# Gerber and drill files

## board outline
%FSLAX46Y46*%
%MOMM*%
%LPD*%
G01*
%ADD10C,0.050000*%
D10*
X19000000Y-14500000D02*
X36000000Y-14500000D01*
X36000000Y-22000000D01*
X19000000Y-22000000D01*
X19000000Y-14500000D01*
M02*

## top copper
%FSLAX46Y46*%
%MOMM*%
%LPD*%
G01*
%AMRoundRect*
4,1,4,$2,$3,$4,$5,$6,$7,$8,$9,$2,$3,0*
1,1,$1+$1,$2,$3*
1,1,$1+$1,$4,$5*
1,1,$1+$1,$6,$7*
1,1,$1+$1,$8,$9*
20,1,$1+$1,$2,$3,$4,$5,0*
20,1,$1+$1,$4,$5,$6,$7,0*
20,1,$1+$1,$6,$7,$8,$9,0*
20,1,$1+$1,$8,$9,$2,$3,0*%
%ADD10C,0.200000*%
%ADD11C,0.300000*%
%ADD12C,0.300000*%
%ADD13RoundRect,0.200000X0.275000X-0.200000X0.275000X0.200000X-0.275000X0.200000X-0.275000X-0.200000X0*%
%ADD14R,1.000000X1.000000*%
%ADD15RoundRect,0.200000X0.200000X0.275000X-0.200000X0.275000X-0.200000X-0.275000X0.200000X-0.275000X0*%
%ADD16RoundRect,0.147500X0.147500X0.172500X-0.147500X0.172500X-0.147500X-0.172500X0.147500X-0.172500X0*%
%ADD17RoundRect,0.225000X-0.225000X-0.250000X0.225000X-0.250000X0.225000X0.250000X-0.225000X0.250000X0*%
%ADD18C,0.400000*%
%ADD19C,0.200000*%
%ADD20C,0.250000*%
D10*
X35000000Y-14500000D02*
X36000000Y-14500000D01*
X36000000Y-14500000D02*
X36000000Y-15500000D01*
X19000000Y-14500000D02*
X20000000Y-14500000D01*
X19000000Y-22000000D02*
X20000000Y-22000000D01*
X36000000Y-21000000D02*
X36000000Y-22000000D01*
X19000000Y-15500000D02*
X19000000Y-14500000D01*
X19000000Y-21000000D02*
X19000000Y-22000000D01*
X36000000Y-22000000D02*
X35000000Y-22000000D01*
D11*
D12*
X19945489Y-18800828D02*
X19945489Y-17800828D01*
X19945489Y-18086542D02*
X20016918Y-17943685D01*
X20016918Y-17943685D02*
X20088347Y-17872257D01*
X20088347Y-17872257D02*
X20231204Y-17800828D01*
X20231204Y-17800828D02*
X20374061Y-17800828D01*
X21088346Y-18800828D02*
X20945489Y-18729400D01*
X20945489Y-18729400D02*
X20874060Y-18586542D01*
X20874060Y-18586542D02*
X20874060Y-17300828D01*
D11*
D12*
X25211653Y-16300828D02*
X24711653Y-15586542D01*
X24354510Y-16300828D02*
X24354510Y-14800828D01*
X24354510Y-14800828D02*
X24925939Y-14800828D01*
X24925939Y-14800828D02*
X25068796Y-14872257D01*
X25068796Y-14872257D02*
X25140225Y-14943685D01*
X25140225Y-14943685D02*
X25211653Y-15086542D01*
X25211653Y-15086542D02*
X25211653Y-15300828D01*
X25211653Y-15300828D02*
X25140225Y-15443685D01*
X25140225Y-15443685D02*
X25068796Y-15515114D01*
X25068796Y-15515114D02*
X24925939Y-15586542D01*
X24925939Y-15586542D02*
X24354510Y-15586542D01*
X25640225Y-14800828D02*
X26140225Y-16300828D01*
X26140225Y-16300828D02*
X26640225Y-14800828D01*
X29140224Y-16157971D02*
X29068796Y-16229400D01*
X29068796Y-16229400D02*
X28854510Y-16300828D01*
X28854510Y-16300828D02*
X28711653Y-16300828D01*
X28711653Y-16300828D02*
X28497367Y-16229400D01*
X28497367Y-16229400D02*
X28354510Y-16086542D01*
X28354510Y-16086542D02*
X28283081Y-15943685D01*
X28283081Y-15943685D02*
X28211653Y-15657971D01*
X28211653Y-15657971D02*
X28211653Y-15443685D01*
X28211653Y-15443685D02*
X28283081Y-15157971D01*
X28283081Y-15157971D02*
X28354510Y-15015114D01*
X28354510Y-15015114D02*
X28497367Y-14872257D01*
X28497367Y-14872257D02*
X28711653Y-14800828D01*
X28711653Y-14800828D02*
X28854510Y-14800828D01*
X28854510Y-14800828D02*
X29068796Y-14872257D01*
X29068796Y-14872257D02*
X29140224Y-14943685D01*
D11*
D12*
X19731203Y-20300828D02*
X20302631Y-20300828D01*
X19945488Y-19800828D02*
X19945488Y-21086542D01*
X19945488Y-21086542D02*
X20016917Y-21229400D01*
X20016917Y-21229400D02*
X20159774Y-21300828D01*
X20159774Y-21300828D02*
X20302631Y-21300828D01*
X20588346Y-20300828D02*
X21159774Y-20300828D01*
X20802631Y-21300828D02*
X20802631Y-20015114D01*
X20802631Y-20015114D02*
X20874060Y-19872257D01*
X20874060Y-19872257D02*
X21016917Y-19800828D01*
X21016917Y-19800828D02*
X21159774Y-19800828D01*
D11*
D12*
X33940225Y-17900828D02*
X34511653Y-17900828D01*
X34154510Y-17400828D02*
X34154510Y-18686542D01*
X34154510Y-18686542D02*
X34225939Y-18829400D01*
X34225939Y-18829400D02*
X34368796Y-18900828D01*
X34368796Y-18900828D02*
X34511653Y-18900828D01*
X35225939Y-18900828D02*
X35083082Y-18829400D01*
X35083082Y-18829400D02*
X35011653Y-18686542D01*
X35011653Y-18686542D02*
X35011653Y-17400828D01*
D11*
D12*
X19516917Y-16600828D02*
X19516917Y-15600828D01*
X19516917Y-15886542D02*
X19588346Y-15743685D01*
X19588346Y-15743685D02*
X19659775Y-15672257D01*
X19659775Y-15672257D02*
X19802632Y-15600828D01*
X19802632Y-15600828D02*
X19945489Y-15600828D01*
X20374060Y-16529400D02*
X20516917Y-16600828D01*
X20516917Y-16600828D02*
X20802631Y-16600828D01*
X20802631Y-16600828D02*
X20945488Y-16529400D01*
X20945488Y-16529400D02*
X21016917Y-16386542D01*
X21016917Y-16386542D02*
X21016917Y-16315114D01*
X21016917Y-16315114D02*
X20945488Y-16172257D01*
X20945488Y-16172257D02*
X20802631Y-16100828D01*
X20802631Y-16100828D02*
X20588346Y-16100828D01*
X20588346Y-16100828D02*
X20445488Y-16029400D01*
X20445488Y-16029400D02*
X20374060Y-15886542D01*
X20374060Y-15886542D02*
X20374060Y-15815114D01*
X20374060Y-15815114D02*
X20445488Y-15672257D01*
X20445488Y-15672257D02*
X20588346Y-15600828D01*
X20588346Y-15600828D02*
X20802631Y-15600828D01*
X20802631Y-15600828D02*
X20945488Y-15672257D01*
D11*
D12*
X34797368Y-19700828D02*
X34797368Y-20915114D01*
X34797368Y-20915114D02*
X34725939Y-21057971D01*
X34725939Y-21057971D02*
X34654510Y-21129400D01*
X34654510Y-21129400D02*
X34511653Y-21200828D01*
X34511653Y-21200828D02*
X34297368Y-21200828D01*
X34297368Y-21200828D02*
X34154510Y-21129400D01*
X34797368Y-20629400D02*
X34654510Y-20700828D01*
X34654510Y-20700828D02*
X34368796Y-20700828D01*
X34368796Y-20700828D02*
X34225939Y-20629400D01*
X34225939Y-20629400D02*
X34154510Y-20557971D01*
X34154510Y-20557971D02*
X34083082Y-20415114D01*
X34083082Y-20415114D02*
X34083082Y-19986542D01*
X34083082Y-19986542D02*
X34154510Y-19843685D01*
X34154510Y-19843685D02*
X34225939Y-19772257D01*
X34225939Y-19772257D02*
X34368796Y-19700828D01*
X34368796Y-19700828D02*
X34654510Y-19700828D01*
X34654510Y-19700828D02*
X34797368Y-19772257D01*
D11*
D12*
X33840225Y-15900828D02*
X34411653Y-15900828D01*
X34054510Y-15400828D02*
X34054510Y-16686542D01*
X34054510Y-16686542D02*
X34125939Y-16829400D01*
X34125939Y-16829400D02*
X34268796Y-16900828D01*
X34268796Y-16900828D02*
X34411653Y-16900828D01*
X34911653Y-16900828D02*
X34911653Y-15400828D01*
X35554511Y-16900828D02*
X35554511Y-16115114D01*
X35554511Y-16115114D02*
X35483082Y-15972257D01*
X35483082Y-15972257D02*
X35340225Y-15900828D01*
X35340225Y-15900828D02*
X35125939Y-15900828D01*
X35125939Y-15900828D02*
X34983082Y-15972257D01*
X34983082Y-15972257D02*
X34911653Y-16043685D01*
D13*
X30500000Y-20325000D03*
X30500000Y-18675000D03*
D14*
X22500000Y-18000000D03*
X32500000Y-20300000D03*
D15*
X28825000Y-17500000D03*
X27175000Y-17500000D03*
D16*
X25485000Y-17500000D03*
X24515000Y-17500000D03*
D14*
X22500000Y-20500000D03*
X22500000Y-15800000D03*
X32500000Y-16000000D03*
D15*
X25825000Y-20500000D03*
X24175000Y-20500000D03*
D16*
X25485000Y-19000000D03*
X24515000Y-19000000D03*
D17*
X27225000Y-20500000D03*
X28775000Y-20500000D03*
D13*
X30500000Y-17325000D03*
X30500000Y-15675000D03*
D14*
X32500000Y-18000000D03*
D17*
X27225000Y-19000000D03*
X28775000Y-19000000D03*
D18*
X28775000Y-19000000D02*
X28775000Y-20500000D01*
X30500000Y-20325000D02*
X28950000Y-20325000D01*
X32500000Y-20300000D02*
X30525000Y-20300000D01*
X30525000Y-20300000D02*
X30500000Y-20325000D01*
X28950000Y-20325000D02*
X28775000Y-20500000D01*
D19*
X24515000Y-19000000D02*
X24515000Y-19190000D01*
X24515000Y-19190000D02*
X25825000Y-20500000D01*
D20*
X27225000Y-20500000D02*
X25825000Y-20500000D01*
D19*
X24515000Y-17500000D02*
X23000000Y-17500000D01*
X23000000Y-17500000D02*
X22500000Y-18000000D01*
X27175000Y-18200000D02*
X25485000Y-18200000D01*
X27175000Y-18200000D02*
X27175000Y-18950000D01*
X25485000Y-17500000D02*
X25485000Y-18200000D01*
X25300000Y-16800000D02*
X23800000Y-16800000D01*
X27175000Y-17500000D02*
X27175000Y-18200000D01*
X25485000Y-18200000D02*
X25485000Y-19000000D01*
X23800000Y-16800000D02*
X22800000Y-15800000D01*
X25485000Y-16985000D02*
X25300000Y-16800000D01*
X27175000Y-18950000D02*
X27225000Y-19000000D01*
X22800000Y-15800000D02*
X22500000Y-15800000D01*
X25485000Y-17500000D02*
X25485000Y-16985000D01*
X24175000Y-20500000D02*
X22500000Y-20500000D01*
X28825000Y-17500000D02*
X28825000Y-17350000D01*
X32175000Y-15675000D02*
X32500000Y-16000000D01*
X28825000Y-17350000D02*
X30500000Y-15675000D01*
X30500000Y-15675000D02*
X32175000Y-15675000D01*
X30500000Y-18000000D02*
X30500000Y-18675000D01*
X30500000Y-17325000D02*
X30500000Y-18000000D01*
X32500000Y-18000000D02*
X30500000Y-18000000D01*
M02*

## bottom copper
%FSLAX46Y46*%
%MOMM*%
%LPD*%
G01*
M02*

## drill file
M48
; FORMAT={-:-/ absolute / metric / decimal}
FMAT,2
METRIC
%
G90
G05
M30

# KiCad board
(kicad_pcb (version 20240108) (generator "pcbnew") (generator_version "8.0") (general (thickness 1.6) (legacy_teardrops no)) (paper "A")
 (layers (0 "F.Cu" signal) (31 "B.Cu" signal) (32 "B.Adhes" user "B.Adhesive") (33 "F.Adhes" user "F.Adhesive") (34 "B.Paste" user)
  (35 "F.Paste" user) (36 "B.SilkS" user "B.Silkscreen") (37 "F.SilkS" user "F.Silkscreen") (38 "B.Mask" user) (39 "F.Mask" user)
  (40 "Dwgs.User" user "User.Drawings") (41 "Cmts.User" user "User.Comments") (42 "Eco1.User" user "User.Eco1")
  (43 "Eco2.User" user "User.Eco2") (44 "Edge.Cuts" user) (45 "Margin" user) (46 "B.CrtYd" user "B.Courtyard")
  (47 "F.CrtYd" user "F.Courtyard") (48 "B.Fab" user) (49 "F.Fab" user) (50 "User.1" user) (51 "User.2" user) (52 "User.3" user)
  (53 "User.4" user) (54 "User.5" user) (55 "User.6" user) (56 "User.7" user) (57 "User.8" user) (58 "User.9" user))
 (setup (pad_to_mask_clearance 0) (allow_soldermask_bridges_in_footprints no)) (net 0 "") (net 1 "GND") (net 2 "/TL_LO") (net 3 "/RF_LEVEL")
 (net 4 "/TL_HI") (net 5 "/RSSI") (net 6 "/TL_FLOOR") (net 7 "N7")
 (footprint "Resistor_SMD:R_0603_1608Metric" (layer "F.Cu") (at 30.5 19.5 90)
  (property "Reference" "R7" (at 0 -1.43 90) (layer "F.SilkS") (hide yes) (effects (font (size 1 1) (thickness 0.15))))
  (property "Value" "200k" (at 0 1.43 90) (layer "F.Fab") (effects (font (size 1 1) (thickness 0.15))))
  (pad "1" smd roundrect (at -0.825 0 90) (size 0.8 0.95) (layers "F.Cu" "F.Paste" "F.Mask") (roundrect_rratio 0.25) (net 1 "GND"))
  (pad "2" smd roundrect (at 0.825 0 90) (size 0.8 0.95) (layers "F.Cu" "F.Paste" "F.Mask") (roundrect_rratio 0.25) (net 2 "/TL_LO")))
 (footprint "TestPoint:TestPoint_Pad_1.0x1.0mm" (layer "F.Cu") (at 22.5 18)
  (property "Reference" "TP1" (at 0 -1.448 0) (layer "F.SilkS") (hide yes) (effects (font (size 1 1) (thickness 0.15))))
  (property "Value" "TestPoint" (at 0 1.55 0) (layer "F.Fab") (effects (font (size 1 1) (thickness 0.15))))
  (pad "1" smd rect (at 0 0) (size 1 1) (layers "F.Cu" "F.Mask") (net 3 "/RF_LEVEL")))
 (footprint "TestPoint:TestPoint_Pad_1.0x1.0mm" (layer "F.Cu") (at 32.5 20.3 90)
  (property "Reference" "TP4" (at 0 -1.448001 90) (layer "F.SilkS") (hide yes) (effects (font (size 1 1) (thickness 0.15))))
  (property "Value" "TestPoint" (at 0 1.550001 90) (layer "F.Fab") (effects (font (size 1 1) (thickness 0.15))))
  (pad "1" smd rect (at 0 0 90) (size 1 1) (layers "F.Cu" "F.Mask") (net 1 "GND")))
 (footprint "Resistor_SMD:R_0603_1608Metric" (layer "F.Cu") (at 28 17.5 180)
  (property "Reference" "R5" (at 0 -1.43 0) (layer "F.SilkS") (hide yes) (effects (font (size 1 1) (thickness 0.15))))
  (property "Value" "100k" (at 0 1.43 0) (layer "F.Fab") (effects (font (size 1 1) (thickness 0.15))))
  (pad "1" smd roundrect (at -0.825 0 180) (size 0.8 0.95) (layers "F.Cu" "F.Paste" "F.Mask") (roundrect_rratio 0.25) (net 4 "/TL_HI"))
  (pad "2" smd roundrect (at 0.825 0 180) (size 0.8 0.95) (layers "F.Cu" "F.Paste" "F.Mask") (roundrect_rratio 0.25) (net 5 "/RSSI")))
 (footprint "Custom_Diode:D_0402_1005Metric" (layer "F.Cu") (at 25 17.5 180)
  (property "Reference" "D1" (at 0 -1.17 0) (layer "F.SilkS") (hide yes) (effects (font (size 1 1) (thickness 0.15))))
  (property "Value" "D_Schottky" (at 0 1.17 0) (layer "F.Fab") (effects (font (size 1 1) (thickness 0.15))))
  (pad "1" smd roundrect (at -0.485 0 180) (size 0.59 0.64) (layers "F.Cu" "F.Paste" "F.Mask") (roundrect_rratio 0.25) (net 5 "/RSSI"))
  (pad "2" smd roundrect (at 0.485 0 180) (size 0.59 0.64) (layers "F.Cu" "F.Paste" "F.Mask") (roundrect_rratio 0.25) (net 3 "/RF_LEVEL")))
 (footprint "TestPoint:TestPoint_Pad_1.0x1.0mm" (layer "F.Cu") (at 22.5 20.5)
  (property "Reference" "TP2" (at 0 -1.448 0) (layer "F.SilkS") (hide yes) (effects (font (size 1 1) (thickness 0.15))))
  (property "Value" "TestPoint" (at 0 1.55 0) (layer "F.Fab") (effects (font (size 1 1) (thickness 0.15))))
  (pad "1" smd rect (at 0 0) (size 1 1) (layers "F.Cu" "F.Mask") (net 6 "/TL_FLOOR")))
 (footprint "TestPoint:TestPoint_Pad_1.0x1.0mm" (layer "F.Cu") (at 22.5 15.8)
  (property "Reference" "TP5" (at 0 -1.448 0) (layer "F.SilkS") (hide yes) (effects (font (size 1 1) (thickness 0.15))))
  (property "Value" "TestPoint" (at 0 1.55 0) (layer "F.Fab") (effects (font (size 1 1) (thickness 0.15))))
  (pad "1" smd rect (at 0 0) (size 1 1) (layers "F.Cu" "F.Mask") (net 5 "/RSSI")))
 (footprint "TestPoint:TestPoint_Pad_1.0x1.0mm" (layer "F.Cu") (at 32.5 16)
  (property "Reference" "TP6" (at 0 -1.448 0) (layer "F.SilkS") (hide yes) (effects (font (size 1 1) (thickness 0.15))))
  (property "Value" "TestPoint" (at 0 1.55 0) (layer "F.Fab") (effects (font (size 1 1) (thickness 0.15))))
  (pad "1" smd rect (at 0 0) (size 1 1) (layers "F.Cu" "F.Mask") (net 4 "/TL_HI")))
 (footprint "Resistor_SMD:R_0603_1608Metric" (layer "F.Cu") (at 25 20.5 180)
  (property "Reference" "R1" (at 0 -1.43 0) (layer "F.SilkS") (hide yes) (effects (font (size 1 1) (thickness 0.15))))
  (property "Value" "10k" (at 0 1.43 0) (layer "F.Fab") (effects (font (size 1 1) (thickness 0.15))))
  (pad "1" smd roundrect (at -0.825 0 180) (size 0.8 0.95) (layers "F.Cu" "F.Paste" "F.Mask") (roundrect_rratio 0.25) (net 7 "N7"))
  (pad "2" smd roundrect (at 0.825 0 180) (size 0.8 0.95) (layers "F.Cu" "F.Paste" "F.Mask") (roundrect_rratio 0.25) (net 6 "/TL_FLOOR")))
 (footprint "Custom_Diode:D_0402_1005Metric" (layer "F.Cu") (at 25 19 180)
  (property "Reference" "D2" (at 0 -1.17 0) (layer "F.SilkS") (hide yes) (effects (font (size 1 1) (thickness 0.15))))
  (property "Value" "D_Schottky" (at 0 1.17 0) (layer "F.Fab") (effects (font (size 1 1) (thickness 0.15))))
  (pad "1" smd roundrect (at -0.485 0 180) (size 0.59 0.64) (layers "F.Cu" "F.Paste" "F.Mask") (roundrect_rratio 0.25) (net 5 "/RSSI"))
  (pad "2" smd roundrect (at 0.485 0 180) (size 0.59 0.64) (layers "F.Cu" "F.Paste" "F.Mask") (roundrect_rratio 0.25) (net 7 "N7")))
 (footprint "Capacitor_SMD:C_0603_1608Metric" (layer "F.Cu") (at 28 20.5)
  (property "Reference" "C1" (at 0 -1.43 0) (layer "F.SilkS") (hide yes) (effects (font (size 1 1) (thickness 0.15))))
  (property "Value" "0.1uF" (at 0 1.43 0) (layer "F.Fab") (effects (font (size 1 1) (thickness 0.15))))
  (pad "1" smd roundrect (at -0.775 0) (size 0.9 0.95) (layers "F.Cu" "F.Paste" "F.Mask") (roundrect_rratio 0.25) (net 7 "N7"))
  (pad "2" smd roundrect (at 0.775 0) (size 0.9 0.95) (layers "F.Cu" "F.Paste" "F.Mask") (roundrect_rratio 0.25) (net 1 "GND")))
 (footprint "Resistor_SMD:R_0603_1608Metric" (layer "F.Cu") (at 30.5 16.5 90)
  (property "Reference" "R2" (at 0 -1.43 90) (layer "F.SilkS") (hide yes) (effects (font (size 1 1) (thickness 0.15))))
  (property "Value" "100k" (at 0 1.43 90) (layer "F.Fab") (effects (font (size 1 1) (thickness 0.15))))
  (pad "1" smd roundrect (at -0.825 0 90) (size 0.8 0.95) (layers "F.Cu" "F.Paste" "F.Mask") (roundrect_rratio 0.25) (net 2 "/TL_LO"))
  (pad "2" smd roundrect (at 0.825 0 90) (size 0.8 0.95) (layers "F.Cu" "F.Paste" "F.Mask") (roundrect_rratio 0.25) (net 4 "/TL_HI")))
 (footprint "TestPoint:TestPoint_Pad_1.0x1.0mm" (layer "F.Cu") (at 32.5 18)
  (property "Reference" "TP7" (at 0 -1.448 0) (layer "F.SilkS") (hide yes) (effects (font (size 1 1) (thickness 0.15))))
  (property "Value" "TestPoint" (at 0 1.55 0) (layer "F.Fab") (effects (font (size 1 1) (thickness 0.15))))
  (pad "1" smd rect (at 0 0) (size 1 1) (layers "F.Cu" "F.Mask") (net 2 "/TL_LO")))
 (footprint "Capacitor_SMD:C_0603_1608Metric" (layer "F.Cu") (at 28 19)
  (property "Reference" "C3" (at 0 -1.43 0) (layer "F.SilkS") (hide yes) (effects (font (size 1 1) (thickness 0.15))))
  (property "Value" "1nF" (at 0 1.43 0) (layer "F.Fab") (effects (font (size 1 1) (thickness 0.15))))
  (pad "1" smd roundrect (at -0.775 0) (size 0.9 0.95) (layers "F.Cu" "F.Paste" "F.Mask") (roundrect_rratio 0.25) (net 5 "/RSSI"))
  (pad "2" smd roundrect (at 0.775 0) (size 0.9 0.95) (layers "F.Cu" "F.Paste" "F.Mask") (roundrect_rratio 0.25) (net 1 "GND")))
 (gr_line (start 35 14.5) (end 36 14.5) (stroke (width 0.2) (type default)) (layer "F.Cu"))
 (gr_line (start 36 14.5) (end 36 15.5) (stroke (width 0.2) (type default)) (layer "F.Cu"))
 (gr_line (start 19 14.5) (end 20 14.5) (stroke (width 0.2) (type default)) (layer "F.Cu"))
 (gr_line (start 19 22) (end 20 22) (stroke (width 0.2) (type default)) (layer "F.Cu"))
 (gr_line (start 36 21) (end 36 22) (stroke (width 0.2) (type default)) (layer "F.Cu"))
 (gr_line (start 19 15.5) (end 19 14.5) (stroke (width 0.2) (type default)) (layer "F.Cu"))
 (gr_line (start 19 21) (end 19 22) (stroke (width 0.2) (type default)) (layer "F.Cu"))
 (gr_line (start 36 22) (end 35 22) (stroke (width 0.2) (type default)) (layer "F.Cu"))
 (gr_rect (start 19 14.5) (end 36 22) (stroke (width 0.05) (type default)) (fill none) (layer "Edge.Cuts"))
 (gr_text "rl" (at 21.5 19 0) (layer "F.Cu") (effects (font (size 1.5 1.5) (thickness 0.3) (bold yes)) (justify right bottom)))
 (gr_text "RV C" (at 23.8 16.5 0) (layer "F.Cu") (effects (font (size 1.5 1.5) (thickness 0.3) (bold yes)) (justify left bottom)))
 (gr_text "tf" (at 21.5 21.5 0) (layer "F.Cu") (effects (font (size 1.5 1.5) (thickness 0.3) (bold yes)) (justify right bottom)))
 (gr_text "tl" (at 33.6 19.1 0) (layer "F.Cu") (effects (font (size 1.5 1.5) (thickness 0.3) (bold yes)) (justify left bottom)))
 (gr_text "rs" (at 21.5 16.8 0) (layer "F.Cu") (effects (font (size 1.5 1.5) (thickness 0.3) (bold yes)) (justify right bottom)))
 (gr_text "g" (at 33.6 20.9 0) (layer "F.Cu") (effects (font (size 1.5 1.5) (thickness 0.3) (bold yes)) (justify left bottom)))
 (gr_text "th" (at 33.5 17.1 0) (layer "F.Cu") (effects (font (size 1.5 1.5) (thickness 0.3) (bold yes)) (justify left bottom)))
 (segment (start 28.775 19) (end 28.775 20.5) (width 0.4) (layer "F.Cu") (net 1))
 (segment (start 30.5 20.325) (end 28.95 20.325) (width 0.4) (layer "F.Cu") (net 1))
 (segment (start 32.5 20.3) (end 30.525 20.3) (width 0.4) (layer "F.Cu") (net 1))
 (segment (start 30.525 20.3) (end 30.5 20.325) (width 0.4) (layer "F.Cu") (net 1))
 (segment (start 28.95 20.325) (end 28.775 20.5) (width 0.4) (layer "F.Cu") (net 1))
 (segment (start 24.515 19) (end 24.515 19.19) (width 0.2) (layer "F.Cu") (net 7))
 (segment (start 24.515 19.19) (end 25.825 20.5) (width 0.2) (layer "F.Cu") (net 7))
 (segment (start 27.225 20.5) (end 25.825 20.5) (width 0.25) (layer "F.Cu") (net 7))
 (segment (start 24.515 17.5) (end 23 17.5) (width 0.2) (layer "F.Cu") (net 3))
 (segment (start 23 17.5) (end 22.5 18) (width 0.2) (layer "F.Cu") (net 3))
 (segment (start 27.175 18.2) (end 25.485 18.2) (width 0.2) (layer "F.Cu") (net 5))
 (segment (start 27.175 18.2) (end 27.175 18.95) (width 0.2) (layer "F.Cu") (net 5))
 (segment (start 25.485 17.5) (end 25.485 18.2) (width 0.2) (layer "F.Cu") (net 5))
 (segment (start 25.3 16.8) (end 23.8 16.8) (width 0.2) (layer "F.Cu") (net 5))
 (segment (start 27.175 17.5) (end 27.175 18.2) (width 0.2) (layer "F.Cu") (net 5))
 (segment (start 25.485 18.2) (end 25.485 19) (width 0.2) (layer "F.Cu") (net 5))
 (segment (start 23.8 16.8) (end 22.8 15.8) (width 0.2) (layer "F.Cu") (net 5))
 (segment (start 25.485 16.985) (end 25.3 16.8) (width 0.2) (layer "F.Cu") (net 5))
 (segment (start 27.175 18.95) (end 27.225 19) (width 0.2) (layer "F.Cu") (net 5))
 (segment (start 22.8 15.8) (end 22.5 15.8) (width 0.2) (layer "F.Cu") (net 5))
 (segment (start 25.485 17.5) (end 25.485 16.985) (width 0.2) (layer "F.Cu") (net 5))
 (segment (start 24.175 20.5) (end 22.5 20.5) (width 0.2) (layer "F.Cu") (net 6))
 (segment (start 28.825 17.5) (end 28.825 17.35) (width 0.2) (layer "F.Cu") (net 4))
 (segment (start 32.175 15.675) (end 32.5 16) (width 0.2) (layer "F.Cu") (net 4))
 (segment (start 28.825 17.35) (end 30.5 15.675) (width 0.2) (layer "F.Cu") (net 4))
 (segment (start 30.5 15.675) (end 32.175 15.675) (width 0.2) (layer "F.Cu") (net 4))
 (segment (start 30.5 18) (end 30.5 18.675) (width 0.2) (layer "F.Cu") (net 2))
 (segment (start 30.5 17.325) (end 30.5 18) (width 0.2) (layer "F.Cu") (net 2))
 (segment (start 32.5 18) (end 30.5 18) (width 0.2) (layer "F.Cu") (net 2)))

